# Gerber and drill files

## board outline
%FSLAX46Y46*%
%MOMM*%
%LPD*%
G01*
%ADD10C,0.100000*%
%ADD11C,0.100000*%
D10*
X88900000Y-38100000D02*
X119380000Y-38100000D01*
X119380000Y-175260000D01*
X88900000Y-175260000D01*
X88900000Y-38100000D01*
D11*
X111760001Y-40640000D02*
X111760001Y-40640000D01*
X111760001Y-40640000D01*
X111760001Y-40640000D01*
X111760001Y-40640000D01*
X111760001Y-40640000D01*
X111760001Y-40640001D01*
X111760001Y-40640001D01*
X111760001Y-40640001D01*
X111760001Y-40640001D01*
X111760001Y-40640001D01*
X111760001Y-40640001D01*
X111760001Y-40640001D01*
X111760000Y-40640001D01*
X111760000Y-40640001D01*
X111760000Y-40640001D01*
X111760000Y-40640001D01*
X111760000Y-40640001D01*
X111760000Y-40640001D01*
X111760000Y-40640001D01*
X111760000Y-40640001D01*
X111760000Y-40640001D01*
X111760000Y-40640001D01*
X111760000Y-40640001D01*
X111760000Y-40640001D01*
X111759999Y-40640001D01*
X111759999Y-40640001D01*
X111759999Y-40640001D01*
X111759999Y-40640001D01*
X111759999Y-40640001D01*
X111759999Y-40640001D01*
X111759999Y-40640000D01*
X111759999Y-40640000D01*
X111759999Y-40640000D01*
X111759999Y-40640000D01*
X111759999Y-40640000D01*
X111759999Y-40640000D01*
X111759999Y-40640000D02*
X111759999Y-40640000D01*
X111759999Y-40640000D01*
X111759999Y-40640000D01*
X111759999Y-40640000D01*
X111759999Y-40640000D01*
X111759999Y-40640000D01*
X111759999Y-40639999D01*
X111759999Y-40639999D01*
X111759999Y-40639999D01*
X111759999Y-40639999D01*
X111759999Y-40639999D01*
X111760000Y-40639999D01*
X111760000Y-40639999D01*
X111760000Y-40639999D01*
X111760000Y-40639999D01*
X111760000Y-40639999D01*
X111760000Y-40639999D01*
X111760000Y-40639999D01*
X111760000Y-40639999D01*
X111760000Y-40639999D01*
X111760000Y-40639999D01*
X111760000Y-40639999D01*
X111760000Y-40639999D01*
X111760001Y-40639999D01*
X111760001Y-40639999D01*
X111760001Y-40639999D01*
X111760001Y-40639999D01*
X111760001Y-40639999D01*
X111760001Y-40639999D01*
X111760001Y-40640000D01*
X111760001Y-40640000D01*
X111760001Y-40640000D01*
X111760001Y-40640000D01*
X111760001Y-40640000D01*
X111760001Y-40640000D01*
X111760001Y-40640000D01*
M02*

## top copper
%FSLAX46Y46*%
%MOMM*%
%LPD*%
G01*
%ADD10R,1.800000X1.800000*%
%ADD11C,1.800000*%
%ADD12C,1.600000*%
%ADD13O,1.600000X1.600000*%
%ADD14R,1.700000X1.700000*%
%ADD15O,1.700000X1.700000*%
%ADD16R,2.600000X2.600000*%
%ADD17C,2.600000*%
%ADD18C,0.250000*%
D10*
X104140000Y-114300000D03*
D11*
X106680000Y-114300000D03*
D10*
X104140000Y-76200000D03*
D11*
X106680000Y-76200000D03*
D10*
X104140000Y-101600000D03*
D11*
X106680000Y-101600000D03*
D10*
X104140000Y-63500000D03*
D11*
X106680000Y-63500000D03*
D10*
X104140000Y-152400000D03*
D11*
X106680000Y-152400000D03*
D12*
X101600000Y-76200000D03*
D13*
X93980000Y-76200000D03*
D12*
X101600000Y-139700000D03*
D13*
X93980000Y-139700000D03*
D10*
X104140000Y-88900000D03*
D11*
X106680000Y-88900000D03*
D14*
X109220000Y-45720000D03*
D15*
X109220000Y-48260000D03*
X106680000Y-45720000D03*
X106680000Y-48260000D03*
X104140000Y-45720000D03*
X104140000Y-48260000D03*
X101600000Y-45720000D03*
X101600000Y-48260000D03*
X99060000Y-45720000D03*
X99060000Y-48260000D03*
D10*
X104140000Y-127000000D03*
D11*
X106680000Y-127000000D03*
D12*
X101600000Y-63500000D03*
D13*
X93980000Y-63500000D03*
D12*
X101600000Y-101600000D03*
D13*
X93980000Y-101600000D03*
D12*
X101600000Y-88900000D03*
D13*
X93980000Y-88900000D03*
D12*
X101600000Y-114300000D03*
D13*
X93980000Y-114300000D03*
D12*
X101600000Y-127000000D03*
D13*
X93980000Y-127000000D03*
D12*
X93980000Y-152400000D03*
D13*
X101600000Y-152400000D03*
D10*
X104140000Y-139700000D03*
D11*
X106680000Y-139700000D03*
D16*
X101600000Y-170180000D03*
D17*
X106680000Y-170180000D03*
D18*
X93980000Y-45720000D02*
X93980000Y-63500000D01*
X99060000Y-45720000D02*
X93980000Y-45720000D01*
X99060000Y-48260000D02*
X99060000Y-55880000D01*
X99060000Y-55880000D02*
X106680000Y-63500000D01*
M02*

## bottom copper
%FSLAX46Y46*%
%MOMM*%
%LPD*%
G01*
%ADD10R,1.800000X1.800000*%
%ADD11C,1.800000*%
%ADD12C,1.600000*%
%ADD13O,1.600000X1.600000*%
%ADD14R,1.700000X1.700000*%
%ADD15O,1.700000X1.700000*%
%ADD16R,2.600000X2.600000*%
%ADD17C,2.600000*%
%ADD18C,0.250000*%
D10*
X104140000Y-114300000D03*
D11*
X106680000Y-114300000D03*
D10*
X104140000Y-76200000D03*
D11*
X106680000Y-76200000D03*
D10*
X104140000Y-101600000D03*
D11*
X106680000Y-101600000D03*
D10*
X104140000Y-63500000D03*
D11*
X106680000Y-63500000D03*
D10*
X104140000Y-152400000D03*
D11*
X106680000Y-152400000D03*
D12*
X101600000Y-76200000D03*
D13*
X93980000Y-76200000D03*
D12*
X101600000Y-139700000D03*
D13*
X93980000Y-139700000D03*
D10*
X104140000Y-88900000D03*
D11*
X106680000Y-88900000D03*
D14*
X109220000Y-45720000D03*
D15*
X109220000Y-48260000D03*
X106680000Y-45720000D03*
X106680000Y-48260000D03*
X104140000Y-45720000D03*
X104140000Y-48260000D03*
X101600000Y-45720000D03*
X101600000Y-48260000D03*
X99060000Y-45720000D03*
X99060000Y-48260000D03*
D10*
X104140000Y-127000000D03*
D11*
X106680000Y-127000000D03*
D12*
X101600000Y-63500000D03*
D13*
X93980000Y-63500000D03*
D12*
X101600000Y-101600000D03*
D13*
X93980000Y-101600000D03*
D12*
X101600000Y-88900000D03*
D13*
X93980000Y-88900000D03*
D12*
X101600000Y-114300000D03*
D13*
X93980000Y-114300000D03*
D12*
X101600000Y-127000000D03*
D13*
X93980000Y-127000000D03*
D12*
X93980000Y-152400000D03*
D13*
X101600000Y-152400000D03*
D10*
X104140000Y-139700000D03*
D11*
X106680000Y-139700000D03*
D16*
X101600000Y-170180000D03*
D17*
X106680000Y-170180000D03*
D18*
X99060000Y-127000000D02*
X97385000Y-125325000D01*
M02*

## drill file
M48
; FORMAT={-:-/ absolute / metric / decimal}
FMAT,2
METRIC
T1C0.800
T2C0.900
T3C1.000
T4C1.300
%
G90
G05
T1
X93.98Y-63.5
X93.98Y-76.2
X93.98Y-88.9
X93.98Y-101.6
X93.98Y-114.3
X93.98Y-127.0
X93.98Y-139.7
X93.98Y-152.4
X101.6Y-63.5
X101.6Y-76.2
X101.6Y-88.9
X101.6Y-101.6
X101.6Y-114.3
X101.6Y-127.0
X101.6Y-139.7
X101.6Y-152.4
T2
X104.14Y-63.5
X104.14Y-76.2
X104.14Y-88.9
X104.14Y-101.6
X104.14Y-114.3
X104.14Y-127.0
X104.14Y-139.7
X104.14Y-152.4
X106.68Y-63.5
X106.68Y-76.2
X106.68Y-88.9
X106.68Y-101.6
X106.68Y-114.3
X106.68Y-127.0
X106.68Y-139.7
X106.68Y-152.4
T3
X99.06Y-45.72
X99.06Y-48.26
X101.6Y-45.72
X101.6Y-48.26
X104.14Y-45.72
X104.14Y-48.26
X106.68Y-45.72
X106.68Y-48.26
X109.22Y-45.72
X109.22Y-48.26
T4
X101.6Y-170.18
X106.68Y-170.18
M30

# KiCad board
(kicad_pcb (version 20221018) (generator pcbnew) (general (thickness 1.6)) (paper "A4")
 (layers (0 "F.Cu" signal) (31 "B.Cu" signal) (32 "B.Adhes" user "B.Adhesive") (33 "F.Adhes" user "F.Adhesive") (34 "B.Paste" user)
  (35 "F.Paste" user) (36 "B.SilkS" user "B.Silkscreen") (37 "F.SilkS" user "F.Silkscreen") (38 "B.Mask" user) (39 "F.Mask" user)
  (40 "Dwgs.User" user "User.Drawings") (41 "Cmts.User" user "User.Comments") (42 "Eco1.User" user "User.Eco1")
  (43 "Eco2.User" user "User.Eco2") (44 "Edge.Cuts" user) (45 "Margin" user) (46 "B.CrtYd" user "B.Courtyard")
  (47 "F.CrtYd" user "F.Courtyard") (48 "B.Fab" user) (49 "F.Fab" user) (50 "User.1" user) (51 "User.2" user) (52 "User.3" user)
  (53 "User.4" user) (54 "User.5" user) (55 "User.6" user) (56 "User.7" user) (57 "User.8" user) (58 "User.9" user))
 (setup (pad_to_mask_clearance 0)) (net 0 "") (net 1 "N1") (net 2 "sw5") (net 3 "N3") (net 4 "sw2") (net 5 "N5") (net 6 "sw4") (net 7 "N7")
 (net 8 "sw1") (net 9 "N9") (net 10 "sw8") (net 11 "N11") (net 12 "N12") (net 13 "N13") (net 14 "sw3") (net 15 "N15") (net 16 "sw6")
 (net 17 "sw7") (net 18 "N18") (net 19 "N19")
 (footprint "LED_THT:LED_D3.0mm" (layer "F.Cu") (at 104.14 114.3)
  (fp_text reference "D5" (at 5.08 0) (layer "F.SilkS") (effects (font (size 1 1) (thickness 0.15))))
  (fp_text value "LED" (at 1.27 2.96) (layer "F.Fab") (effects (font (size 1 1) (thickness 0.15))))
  (pad "1" thru_hole rect (at 0 0) (size 1.8 1.8) (drill 0.9) (layers "*.Cu" "*.Mask") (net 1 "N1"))
  (pad "2" thru_hole circle (at 2.54 0) (size 1.8 1.8) (drill 0.9) (layers "*.Cu" "*.Mask") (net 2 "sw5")))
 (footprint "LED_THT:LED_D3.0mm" (layer "F.Cu") (at 104.14 76.2)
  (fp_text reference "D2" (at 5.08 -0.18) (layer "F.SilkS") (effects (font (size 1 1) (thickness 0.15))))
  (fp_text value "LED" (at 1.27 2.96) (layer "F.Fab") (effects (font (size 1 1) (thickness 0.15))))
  (pad "1" thru_hole rect (at 0 0) (size 1.8 1.8) (drill 0.9) (layers "*.Cu" "*.Mask") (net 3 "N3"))
  (pad "2" thru_hole circle (at 2.54 0) (size 1.8 1.8) (drill 0.9) (layers "*.Cu" "*.Mask") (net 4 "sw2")))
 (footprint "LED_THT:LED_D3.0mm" (layer "F.Cu") (at 104.14 101.6)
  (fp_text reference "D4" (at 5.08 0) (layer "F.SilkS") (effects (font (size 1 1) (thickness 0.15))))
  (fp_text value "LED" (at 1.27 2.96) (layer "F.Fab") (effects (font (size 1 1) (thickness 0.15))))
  (pad "1" thru_hole rect (at 0 0) (size 1.8 1.8) (drill 0.9) (layers "*.Cu" "*.Mask") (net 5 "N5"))
  (pad "2" thru_hole circle (at 2.54 0) (size 1.8 1.8) (drill 0.9) (layers "*.Cu" "*.Mask") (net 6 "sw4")))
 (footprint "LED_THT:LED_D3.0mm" (layer "F.Cu") (at 104.14 63.5)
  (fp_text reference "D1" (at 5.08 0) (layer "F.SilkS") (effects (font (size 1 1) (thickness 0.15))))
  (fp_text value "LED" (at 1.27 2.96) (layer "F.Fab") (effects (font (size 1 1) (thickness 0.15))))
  (pad "1" thru_hole rect (at 0 0) (size 1.8 1.8) (drill 0.9) (layers "*.Cu" "*.Mask") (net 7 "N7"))
  (pad "2" thru_hole circle (at 2.54 0) (size 1.8 1.8) (drill 0.9) (layers "*.Cu" "*.Mask") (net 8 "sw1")))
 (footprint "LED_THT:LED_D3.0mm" (layer "F.Cu") (at 104.14 152.4)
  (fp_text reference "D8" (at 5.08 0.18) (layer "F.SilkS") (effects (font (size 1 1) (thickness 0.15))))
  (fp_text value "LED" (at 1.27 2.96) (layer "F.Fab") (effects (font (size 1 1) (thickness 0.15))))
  (pad "1" thru_hole rect (at 0 0) (size 1.8 1.8) (drill 0.9) (layers "*.Cu" "*.Mask") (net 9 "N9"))
  (pad "2" thru_hole circle (at 2.54 0) (size 1.8 1.8) (drill 0.9) (layers "*.Cu" "*.Mask") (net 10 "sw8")))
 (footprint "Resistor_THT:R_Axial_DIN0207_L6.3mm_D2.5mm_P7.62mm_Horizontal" (layer "F.Cu") (at 101.6 76.2 180)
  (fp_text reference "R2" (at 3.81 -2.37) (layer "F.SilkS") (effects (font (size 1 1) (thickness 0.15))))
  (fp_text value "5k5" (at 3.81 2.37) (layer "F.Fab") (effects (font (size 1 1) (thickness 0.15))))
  (pad "1" thru_hole circle (at 0 0 180) (size 1.6 1.6) (drill 0.8) (layers "*.Cu" "*.Mask") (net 3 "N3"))
  (pad "2" thru_hole oval (at 7.62 0 180) (size 1.6 1.6) (drill 0.8) (layers "*.Cu" "*.Mask") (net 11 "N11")))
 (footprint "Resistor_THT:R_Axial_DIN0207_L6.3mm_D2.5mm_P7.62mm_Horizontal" (layer "F.Cu") (at 101.6 139.7 180)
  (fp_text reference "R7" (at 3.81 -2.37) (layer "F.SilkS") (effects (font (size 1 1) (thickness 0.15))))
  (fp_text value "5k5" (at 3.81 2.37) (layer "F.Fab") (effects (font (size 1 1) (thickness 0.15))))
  (pad "1" thru_hole circle (at 0 0 180) (size 1.6 1.6) (drill 0.8) (layers "*.Cu" "*.Mask") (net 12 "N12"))
  (pad "2" thru_hole oval (at 7.62 0 180) (size 1.6 1.6) (drill 0.8) (layers "*.Cu" "*.Mask") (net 11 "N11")))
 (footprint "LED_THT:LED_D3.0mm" (layer "F.Cu") (at 104.14 88.9)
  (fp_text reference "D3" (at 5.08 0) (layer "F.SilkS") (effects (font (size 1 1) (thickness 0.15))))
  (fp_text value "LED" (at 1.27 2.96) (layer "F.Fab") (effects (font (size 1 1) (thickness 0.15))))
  (pad "1" thru_hole rect (at 0 0) (size 1.8 1.8) (drill 0.9) (layers "*.Cu" "*.Mask") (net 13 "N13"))
  (pad "2" thru_hole circle (at 2.54 0) (size 1.8 1.8) (drill 0.9) (layers "*.Cu" "*.Mask") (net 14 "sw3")))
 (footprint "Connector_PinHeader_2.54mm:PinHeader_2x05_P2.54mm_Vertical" (layer "F.Cu") (at 109.22 45.72 -90)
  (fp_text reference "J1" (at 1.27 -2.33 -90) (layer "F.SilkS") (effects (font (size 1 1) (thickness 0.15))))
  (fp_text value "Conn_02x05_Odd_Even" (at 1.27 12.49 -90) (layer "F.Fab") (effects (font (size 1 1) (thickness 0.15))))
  (pad "1" thru_hole rect (at 0 0 270) (size 1.7 1.7) (drill 1) (layers "*.Cu" "*.Mask") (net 10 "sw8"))
  (pad "2" thru_hole oval (at 2.54 0 270) (size 1.7 1.7) (drill 1) (layers "*.Cu" "*.Mask") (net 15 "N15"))
  (pad "3" thru_hole oval (at 0 2.54 270) (size 1.7 1.7) (drill 1) (layers "*.Cu" "*.Mask") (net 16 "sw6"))
  (pad "4" thru_hole oval (at 2.54 2.54 270) (size 1.7 1.7) (drill 1) (layers "*.Cu" "*.Mask") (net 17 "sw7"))
  (pad "5" thru_hole oval (at 0 5.08 270) (size 1.7 1.7) (drill 1) (layers "*.Cu" "*.Mask") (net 6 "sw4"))
  (pad "6" thru_hole oval (at 2.54 5.08 270) (size 1.7 1.7) (drill 1) (layers "*.Cu" "*.Mask") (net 2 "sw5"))
  (pad "7" thru_hole oval (at 0 7.62 270) (size 1.7 1.7) (drill 1) (layers "*.Cu" "*.Mask") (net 4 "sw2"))
  (pad "8" thru_hole oval (at 2.54 7.62 270) (size 1.7 1.7) (drill 1) (layers "*.Cu" "*.Mask") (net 14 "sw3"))
  (pad "9" thru_hole oval (at 0 10.16 270) (size 1.7 1.7) (drill 1) (layers "*.Cu" "*.Mask") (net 11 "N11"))
  (pad "10" thru_hole oval (at 2.54 10.16 270) (size 1.7 1.7) (drill 1) (layers "*.Cu" "*.Mask") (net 8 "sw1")))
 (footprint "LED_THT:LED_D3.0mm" (layer "F.Cu") (at 104.14 127)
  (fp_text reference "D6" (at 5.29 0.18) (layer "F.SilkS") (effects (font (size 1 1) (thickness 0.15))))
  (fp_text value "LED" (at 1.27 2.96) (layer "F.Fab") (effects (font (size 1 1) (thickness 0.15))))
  (pad "1" thru_hole rect (at 0 0) (size 1.8 1.8) (drill 0.9) (layers "*.Cu" "*.Mask") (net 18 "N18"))
  (pad "2" thru_hole circle (at 2.54 0) (size 1.8 1.8) (drill 0.9) (layers "*.Cu" "*.Mask") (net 16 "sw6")))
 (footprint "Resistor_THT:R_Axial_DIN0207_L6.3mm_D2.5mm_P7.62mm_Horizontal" (layer "F.Cu") (at 101.6 63.5 180)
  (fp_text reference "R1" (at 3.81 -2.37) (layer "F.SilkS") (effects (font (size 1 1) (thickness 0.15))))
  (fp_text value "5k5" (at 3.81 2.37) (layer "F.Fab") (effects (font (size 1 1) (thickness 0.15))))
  (pad "1" thru_hole circle (at 0 0 180) (size 1.6 1.6) (drill 0.8) (layers "*.Cu" "*.Mask") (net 7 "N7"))
  (pad "2" thru_hole oval (at 7.62 0 180) (size 1.6 1.6) (drill 0.8) (layers "*.Cu" "*.Mask") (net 11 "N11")))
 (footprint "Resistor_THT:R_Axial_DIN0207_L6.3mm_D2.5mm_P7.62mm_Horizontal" (layer "F.Cu") (at 101.6 101.6 180)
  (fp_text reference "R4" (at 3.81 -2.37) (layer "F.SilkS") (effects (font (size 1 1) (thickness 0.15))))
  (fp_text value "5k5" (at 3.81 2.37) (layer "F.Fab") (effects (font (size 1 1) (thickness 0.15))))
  (pad "1" thru_hole circle (at 0 0 180) (size 1.6 1.6) (drill 0.8) (layers "*.Cu" "*.Mask") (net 5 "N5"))
  (pad "2" thru_hole oval (at 7.62 0 180) (size 1.6 1.6) (drill 0.8) (layers "*.Cu" "*.Mask") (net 11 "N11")))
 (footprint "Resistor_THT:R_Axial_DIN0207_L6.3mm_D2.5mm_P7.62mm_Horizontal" (layer "F.Cu") (at 101.6 88.9 180)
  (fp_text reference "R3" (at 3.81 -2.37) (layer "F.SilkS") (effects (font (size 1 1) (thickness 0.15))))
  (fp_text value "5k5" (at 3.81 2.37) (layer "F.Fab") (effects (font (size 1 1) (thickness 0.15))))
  (pad "1" thru_hole circle (at 0 0 180) (size 1.6 1.6) (drill 0.8) (layers "*.Cu" "*.Mask") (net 13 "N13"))
  (pad "2" thru_hole oval (at 7.62 0 180) (size 1.6 1.6) (drill 0.8) (layers "*.Cu" "*.Mask") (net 11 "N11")))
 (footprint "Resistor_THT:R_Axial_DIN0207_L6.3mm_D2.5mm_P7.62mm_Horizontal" (layer "F.Cu") (at 101.6 114.3 180)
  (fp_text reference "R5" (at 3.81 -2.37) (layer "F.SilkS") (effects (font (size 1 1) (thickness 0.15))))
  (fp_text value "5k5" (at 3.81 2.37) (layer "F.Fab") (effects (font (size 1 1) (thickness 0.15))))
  (pad "1" thru_hole circle (at 0 0 180) (size 1.6 1.6) (drill 0.8) (layers "*.Cu" "*.Mask") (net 1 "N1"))
  (pad "2" thru_hole oval (at 7.62 0 180) (size 1.6 1.6) (drill 0.8) (layers "*.Cu" "*.Mask") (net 11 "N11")))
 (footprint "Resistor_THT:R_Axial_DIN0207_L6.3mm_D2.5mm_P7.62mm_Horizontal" (layer "F.Cu") (at 101.6 127 180)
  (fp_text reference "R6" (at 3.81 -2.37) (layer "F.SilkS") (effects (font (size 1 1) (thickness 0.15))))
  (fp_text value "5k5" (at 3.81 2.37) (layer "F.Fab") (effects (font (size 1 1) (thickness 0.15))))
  (pad "1" thru_hole circle (at 0 0 180) (size 1.6 1.6) (drill 0.8) (layers "*.Cu" "*.Mask") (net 18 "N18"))
  (pad "2" thru_hole oval (at 7.62 0 180) (size 1.6 1.6) (drill 0.8) (layers "*.Cu" "*.Mask") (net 11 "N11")))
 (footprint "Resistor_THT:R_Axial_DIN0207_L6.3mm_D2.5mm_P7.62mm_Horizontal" (layer "F.Cu") (at 93.98 152.4)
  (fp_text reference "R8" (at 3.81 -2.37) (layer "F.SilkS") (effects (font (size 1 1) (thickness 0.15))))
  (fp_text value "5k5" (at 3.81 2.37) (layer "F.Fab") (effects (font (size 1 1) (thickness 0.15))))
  (pad "1" thru_hole circle (at 0 0) (size 1.6 1.6) (drill 0.8) (layers "*.Cu" "*.Mask") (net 9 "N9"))
  (pad "2" thru_hole oval (at 7.62 0) (size 1.6 1.6) (drill 0.8) (layers "*.Cu" "*.Mask") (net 11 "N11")))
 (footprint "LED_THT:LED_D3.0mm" (layer "F.Cu") (at 104.14 139.7)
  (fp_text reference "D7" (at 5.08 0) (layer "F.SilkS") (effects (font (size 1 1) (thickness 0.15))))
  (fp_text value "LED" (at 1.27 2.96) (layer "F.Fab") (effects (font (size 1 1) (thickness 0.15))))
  (pad "1" thru_hole rect (at 0 0) (size 1.8 1.8) (drill 0.9) (layers "*.Cu" "*.Mask") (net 12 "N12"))
  (pad "2" thru_hole circle (at 2.54 0) (size 1.8 1.8) (drill 0.9) (layers "*.Cu" "*.Mask") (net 17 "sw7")))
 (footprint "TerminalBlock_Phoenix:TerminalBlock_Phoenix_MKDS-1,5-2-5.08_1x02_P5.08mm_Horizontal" (layer "F.Cu") (at 101.6 170.18)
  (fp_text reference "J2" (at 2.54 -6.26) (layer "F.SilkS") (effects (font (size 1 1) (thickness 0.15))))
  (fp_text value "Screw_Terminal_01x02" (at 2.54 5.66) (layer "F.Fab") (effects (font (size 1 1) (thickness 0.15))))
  (pad "1" thru_hole rect (at 0 0) (size 2.6 2.6) (drill 1.3) (layers "*.Cu" "*.Mask") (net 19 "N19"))
  (pad "2" thru_hole circle (at 5.08 0) (size 2.6 2.6) (drill 1.3) (layers "*.Cu" "*.Mask") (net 11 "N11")))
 (gr_rect (start 88.9 38.1) (end 119.38 175.26) (stroke (width 0.1) (type default)) (fill none) (layer "Edge.Cuts"))
 (gr_circle (center 111.76 40.64) (end 111.76 40.64) (stroke (width 0.1) (type default)) (fill none) (layer "Edge.Cuts"))
 (segment (start 99.06 127) (end 97.385 125.325) (width 0.25) (layer "B.Cu") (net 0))
 (segment (start 93.98 45.72) (end 93.98 63.5) (width 0.25) (layer "F.Cu") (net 11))
 (segment (start 99.06 45.72) (end 93.98 45.72) (width 0.25) (layer "F.Cu") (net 11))
 (segment (start 99.06 48.26) (end 99.06 55.88) (width 0.25) (layer "F.Cu") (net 8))
 (segment (start 99.06 55.88) (end 106.68 63.5) (width 0.25) (layer "F.Cu") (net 8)))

